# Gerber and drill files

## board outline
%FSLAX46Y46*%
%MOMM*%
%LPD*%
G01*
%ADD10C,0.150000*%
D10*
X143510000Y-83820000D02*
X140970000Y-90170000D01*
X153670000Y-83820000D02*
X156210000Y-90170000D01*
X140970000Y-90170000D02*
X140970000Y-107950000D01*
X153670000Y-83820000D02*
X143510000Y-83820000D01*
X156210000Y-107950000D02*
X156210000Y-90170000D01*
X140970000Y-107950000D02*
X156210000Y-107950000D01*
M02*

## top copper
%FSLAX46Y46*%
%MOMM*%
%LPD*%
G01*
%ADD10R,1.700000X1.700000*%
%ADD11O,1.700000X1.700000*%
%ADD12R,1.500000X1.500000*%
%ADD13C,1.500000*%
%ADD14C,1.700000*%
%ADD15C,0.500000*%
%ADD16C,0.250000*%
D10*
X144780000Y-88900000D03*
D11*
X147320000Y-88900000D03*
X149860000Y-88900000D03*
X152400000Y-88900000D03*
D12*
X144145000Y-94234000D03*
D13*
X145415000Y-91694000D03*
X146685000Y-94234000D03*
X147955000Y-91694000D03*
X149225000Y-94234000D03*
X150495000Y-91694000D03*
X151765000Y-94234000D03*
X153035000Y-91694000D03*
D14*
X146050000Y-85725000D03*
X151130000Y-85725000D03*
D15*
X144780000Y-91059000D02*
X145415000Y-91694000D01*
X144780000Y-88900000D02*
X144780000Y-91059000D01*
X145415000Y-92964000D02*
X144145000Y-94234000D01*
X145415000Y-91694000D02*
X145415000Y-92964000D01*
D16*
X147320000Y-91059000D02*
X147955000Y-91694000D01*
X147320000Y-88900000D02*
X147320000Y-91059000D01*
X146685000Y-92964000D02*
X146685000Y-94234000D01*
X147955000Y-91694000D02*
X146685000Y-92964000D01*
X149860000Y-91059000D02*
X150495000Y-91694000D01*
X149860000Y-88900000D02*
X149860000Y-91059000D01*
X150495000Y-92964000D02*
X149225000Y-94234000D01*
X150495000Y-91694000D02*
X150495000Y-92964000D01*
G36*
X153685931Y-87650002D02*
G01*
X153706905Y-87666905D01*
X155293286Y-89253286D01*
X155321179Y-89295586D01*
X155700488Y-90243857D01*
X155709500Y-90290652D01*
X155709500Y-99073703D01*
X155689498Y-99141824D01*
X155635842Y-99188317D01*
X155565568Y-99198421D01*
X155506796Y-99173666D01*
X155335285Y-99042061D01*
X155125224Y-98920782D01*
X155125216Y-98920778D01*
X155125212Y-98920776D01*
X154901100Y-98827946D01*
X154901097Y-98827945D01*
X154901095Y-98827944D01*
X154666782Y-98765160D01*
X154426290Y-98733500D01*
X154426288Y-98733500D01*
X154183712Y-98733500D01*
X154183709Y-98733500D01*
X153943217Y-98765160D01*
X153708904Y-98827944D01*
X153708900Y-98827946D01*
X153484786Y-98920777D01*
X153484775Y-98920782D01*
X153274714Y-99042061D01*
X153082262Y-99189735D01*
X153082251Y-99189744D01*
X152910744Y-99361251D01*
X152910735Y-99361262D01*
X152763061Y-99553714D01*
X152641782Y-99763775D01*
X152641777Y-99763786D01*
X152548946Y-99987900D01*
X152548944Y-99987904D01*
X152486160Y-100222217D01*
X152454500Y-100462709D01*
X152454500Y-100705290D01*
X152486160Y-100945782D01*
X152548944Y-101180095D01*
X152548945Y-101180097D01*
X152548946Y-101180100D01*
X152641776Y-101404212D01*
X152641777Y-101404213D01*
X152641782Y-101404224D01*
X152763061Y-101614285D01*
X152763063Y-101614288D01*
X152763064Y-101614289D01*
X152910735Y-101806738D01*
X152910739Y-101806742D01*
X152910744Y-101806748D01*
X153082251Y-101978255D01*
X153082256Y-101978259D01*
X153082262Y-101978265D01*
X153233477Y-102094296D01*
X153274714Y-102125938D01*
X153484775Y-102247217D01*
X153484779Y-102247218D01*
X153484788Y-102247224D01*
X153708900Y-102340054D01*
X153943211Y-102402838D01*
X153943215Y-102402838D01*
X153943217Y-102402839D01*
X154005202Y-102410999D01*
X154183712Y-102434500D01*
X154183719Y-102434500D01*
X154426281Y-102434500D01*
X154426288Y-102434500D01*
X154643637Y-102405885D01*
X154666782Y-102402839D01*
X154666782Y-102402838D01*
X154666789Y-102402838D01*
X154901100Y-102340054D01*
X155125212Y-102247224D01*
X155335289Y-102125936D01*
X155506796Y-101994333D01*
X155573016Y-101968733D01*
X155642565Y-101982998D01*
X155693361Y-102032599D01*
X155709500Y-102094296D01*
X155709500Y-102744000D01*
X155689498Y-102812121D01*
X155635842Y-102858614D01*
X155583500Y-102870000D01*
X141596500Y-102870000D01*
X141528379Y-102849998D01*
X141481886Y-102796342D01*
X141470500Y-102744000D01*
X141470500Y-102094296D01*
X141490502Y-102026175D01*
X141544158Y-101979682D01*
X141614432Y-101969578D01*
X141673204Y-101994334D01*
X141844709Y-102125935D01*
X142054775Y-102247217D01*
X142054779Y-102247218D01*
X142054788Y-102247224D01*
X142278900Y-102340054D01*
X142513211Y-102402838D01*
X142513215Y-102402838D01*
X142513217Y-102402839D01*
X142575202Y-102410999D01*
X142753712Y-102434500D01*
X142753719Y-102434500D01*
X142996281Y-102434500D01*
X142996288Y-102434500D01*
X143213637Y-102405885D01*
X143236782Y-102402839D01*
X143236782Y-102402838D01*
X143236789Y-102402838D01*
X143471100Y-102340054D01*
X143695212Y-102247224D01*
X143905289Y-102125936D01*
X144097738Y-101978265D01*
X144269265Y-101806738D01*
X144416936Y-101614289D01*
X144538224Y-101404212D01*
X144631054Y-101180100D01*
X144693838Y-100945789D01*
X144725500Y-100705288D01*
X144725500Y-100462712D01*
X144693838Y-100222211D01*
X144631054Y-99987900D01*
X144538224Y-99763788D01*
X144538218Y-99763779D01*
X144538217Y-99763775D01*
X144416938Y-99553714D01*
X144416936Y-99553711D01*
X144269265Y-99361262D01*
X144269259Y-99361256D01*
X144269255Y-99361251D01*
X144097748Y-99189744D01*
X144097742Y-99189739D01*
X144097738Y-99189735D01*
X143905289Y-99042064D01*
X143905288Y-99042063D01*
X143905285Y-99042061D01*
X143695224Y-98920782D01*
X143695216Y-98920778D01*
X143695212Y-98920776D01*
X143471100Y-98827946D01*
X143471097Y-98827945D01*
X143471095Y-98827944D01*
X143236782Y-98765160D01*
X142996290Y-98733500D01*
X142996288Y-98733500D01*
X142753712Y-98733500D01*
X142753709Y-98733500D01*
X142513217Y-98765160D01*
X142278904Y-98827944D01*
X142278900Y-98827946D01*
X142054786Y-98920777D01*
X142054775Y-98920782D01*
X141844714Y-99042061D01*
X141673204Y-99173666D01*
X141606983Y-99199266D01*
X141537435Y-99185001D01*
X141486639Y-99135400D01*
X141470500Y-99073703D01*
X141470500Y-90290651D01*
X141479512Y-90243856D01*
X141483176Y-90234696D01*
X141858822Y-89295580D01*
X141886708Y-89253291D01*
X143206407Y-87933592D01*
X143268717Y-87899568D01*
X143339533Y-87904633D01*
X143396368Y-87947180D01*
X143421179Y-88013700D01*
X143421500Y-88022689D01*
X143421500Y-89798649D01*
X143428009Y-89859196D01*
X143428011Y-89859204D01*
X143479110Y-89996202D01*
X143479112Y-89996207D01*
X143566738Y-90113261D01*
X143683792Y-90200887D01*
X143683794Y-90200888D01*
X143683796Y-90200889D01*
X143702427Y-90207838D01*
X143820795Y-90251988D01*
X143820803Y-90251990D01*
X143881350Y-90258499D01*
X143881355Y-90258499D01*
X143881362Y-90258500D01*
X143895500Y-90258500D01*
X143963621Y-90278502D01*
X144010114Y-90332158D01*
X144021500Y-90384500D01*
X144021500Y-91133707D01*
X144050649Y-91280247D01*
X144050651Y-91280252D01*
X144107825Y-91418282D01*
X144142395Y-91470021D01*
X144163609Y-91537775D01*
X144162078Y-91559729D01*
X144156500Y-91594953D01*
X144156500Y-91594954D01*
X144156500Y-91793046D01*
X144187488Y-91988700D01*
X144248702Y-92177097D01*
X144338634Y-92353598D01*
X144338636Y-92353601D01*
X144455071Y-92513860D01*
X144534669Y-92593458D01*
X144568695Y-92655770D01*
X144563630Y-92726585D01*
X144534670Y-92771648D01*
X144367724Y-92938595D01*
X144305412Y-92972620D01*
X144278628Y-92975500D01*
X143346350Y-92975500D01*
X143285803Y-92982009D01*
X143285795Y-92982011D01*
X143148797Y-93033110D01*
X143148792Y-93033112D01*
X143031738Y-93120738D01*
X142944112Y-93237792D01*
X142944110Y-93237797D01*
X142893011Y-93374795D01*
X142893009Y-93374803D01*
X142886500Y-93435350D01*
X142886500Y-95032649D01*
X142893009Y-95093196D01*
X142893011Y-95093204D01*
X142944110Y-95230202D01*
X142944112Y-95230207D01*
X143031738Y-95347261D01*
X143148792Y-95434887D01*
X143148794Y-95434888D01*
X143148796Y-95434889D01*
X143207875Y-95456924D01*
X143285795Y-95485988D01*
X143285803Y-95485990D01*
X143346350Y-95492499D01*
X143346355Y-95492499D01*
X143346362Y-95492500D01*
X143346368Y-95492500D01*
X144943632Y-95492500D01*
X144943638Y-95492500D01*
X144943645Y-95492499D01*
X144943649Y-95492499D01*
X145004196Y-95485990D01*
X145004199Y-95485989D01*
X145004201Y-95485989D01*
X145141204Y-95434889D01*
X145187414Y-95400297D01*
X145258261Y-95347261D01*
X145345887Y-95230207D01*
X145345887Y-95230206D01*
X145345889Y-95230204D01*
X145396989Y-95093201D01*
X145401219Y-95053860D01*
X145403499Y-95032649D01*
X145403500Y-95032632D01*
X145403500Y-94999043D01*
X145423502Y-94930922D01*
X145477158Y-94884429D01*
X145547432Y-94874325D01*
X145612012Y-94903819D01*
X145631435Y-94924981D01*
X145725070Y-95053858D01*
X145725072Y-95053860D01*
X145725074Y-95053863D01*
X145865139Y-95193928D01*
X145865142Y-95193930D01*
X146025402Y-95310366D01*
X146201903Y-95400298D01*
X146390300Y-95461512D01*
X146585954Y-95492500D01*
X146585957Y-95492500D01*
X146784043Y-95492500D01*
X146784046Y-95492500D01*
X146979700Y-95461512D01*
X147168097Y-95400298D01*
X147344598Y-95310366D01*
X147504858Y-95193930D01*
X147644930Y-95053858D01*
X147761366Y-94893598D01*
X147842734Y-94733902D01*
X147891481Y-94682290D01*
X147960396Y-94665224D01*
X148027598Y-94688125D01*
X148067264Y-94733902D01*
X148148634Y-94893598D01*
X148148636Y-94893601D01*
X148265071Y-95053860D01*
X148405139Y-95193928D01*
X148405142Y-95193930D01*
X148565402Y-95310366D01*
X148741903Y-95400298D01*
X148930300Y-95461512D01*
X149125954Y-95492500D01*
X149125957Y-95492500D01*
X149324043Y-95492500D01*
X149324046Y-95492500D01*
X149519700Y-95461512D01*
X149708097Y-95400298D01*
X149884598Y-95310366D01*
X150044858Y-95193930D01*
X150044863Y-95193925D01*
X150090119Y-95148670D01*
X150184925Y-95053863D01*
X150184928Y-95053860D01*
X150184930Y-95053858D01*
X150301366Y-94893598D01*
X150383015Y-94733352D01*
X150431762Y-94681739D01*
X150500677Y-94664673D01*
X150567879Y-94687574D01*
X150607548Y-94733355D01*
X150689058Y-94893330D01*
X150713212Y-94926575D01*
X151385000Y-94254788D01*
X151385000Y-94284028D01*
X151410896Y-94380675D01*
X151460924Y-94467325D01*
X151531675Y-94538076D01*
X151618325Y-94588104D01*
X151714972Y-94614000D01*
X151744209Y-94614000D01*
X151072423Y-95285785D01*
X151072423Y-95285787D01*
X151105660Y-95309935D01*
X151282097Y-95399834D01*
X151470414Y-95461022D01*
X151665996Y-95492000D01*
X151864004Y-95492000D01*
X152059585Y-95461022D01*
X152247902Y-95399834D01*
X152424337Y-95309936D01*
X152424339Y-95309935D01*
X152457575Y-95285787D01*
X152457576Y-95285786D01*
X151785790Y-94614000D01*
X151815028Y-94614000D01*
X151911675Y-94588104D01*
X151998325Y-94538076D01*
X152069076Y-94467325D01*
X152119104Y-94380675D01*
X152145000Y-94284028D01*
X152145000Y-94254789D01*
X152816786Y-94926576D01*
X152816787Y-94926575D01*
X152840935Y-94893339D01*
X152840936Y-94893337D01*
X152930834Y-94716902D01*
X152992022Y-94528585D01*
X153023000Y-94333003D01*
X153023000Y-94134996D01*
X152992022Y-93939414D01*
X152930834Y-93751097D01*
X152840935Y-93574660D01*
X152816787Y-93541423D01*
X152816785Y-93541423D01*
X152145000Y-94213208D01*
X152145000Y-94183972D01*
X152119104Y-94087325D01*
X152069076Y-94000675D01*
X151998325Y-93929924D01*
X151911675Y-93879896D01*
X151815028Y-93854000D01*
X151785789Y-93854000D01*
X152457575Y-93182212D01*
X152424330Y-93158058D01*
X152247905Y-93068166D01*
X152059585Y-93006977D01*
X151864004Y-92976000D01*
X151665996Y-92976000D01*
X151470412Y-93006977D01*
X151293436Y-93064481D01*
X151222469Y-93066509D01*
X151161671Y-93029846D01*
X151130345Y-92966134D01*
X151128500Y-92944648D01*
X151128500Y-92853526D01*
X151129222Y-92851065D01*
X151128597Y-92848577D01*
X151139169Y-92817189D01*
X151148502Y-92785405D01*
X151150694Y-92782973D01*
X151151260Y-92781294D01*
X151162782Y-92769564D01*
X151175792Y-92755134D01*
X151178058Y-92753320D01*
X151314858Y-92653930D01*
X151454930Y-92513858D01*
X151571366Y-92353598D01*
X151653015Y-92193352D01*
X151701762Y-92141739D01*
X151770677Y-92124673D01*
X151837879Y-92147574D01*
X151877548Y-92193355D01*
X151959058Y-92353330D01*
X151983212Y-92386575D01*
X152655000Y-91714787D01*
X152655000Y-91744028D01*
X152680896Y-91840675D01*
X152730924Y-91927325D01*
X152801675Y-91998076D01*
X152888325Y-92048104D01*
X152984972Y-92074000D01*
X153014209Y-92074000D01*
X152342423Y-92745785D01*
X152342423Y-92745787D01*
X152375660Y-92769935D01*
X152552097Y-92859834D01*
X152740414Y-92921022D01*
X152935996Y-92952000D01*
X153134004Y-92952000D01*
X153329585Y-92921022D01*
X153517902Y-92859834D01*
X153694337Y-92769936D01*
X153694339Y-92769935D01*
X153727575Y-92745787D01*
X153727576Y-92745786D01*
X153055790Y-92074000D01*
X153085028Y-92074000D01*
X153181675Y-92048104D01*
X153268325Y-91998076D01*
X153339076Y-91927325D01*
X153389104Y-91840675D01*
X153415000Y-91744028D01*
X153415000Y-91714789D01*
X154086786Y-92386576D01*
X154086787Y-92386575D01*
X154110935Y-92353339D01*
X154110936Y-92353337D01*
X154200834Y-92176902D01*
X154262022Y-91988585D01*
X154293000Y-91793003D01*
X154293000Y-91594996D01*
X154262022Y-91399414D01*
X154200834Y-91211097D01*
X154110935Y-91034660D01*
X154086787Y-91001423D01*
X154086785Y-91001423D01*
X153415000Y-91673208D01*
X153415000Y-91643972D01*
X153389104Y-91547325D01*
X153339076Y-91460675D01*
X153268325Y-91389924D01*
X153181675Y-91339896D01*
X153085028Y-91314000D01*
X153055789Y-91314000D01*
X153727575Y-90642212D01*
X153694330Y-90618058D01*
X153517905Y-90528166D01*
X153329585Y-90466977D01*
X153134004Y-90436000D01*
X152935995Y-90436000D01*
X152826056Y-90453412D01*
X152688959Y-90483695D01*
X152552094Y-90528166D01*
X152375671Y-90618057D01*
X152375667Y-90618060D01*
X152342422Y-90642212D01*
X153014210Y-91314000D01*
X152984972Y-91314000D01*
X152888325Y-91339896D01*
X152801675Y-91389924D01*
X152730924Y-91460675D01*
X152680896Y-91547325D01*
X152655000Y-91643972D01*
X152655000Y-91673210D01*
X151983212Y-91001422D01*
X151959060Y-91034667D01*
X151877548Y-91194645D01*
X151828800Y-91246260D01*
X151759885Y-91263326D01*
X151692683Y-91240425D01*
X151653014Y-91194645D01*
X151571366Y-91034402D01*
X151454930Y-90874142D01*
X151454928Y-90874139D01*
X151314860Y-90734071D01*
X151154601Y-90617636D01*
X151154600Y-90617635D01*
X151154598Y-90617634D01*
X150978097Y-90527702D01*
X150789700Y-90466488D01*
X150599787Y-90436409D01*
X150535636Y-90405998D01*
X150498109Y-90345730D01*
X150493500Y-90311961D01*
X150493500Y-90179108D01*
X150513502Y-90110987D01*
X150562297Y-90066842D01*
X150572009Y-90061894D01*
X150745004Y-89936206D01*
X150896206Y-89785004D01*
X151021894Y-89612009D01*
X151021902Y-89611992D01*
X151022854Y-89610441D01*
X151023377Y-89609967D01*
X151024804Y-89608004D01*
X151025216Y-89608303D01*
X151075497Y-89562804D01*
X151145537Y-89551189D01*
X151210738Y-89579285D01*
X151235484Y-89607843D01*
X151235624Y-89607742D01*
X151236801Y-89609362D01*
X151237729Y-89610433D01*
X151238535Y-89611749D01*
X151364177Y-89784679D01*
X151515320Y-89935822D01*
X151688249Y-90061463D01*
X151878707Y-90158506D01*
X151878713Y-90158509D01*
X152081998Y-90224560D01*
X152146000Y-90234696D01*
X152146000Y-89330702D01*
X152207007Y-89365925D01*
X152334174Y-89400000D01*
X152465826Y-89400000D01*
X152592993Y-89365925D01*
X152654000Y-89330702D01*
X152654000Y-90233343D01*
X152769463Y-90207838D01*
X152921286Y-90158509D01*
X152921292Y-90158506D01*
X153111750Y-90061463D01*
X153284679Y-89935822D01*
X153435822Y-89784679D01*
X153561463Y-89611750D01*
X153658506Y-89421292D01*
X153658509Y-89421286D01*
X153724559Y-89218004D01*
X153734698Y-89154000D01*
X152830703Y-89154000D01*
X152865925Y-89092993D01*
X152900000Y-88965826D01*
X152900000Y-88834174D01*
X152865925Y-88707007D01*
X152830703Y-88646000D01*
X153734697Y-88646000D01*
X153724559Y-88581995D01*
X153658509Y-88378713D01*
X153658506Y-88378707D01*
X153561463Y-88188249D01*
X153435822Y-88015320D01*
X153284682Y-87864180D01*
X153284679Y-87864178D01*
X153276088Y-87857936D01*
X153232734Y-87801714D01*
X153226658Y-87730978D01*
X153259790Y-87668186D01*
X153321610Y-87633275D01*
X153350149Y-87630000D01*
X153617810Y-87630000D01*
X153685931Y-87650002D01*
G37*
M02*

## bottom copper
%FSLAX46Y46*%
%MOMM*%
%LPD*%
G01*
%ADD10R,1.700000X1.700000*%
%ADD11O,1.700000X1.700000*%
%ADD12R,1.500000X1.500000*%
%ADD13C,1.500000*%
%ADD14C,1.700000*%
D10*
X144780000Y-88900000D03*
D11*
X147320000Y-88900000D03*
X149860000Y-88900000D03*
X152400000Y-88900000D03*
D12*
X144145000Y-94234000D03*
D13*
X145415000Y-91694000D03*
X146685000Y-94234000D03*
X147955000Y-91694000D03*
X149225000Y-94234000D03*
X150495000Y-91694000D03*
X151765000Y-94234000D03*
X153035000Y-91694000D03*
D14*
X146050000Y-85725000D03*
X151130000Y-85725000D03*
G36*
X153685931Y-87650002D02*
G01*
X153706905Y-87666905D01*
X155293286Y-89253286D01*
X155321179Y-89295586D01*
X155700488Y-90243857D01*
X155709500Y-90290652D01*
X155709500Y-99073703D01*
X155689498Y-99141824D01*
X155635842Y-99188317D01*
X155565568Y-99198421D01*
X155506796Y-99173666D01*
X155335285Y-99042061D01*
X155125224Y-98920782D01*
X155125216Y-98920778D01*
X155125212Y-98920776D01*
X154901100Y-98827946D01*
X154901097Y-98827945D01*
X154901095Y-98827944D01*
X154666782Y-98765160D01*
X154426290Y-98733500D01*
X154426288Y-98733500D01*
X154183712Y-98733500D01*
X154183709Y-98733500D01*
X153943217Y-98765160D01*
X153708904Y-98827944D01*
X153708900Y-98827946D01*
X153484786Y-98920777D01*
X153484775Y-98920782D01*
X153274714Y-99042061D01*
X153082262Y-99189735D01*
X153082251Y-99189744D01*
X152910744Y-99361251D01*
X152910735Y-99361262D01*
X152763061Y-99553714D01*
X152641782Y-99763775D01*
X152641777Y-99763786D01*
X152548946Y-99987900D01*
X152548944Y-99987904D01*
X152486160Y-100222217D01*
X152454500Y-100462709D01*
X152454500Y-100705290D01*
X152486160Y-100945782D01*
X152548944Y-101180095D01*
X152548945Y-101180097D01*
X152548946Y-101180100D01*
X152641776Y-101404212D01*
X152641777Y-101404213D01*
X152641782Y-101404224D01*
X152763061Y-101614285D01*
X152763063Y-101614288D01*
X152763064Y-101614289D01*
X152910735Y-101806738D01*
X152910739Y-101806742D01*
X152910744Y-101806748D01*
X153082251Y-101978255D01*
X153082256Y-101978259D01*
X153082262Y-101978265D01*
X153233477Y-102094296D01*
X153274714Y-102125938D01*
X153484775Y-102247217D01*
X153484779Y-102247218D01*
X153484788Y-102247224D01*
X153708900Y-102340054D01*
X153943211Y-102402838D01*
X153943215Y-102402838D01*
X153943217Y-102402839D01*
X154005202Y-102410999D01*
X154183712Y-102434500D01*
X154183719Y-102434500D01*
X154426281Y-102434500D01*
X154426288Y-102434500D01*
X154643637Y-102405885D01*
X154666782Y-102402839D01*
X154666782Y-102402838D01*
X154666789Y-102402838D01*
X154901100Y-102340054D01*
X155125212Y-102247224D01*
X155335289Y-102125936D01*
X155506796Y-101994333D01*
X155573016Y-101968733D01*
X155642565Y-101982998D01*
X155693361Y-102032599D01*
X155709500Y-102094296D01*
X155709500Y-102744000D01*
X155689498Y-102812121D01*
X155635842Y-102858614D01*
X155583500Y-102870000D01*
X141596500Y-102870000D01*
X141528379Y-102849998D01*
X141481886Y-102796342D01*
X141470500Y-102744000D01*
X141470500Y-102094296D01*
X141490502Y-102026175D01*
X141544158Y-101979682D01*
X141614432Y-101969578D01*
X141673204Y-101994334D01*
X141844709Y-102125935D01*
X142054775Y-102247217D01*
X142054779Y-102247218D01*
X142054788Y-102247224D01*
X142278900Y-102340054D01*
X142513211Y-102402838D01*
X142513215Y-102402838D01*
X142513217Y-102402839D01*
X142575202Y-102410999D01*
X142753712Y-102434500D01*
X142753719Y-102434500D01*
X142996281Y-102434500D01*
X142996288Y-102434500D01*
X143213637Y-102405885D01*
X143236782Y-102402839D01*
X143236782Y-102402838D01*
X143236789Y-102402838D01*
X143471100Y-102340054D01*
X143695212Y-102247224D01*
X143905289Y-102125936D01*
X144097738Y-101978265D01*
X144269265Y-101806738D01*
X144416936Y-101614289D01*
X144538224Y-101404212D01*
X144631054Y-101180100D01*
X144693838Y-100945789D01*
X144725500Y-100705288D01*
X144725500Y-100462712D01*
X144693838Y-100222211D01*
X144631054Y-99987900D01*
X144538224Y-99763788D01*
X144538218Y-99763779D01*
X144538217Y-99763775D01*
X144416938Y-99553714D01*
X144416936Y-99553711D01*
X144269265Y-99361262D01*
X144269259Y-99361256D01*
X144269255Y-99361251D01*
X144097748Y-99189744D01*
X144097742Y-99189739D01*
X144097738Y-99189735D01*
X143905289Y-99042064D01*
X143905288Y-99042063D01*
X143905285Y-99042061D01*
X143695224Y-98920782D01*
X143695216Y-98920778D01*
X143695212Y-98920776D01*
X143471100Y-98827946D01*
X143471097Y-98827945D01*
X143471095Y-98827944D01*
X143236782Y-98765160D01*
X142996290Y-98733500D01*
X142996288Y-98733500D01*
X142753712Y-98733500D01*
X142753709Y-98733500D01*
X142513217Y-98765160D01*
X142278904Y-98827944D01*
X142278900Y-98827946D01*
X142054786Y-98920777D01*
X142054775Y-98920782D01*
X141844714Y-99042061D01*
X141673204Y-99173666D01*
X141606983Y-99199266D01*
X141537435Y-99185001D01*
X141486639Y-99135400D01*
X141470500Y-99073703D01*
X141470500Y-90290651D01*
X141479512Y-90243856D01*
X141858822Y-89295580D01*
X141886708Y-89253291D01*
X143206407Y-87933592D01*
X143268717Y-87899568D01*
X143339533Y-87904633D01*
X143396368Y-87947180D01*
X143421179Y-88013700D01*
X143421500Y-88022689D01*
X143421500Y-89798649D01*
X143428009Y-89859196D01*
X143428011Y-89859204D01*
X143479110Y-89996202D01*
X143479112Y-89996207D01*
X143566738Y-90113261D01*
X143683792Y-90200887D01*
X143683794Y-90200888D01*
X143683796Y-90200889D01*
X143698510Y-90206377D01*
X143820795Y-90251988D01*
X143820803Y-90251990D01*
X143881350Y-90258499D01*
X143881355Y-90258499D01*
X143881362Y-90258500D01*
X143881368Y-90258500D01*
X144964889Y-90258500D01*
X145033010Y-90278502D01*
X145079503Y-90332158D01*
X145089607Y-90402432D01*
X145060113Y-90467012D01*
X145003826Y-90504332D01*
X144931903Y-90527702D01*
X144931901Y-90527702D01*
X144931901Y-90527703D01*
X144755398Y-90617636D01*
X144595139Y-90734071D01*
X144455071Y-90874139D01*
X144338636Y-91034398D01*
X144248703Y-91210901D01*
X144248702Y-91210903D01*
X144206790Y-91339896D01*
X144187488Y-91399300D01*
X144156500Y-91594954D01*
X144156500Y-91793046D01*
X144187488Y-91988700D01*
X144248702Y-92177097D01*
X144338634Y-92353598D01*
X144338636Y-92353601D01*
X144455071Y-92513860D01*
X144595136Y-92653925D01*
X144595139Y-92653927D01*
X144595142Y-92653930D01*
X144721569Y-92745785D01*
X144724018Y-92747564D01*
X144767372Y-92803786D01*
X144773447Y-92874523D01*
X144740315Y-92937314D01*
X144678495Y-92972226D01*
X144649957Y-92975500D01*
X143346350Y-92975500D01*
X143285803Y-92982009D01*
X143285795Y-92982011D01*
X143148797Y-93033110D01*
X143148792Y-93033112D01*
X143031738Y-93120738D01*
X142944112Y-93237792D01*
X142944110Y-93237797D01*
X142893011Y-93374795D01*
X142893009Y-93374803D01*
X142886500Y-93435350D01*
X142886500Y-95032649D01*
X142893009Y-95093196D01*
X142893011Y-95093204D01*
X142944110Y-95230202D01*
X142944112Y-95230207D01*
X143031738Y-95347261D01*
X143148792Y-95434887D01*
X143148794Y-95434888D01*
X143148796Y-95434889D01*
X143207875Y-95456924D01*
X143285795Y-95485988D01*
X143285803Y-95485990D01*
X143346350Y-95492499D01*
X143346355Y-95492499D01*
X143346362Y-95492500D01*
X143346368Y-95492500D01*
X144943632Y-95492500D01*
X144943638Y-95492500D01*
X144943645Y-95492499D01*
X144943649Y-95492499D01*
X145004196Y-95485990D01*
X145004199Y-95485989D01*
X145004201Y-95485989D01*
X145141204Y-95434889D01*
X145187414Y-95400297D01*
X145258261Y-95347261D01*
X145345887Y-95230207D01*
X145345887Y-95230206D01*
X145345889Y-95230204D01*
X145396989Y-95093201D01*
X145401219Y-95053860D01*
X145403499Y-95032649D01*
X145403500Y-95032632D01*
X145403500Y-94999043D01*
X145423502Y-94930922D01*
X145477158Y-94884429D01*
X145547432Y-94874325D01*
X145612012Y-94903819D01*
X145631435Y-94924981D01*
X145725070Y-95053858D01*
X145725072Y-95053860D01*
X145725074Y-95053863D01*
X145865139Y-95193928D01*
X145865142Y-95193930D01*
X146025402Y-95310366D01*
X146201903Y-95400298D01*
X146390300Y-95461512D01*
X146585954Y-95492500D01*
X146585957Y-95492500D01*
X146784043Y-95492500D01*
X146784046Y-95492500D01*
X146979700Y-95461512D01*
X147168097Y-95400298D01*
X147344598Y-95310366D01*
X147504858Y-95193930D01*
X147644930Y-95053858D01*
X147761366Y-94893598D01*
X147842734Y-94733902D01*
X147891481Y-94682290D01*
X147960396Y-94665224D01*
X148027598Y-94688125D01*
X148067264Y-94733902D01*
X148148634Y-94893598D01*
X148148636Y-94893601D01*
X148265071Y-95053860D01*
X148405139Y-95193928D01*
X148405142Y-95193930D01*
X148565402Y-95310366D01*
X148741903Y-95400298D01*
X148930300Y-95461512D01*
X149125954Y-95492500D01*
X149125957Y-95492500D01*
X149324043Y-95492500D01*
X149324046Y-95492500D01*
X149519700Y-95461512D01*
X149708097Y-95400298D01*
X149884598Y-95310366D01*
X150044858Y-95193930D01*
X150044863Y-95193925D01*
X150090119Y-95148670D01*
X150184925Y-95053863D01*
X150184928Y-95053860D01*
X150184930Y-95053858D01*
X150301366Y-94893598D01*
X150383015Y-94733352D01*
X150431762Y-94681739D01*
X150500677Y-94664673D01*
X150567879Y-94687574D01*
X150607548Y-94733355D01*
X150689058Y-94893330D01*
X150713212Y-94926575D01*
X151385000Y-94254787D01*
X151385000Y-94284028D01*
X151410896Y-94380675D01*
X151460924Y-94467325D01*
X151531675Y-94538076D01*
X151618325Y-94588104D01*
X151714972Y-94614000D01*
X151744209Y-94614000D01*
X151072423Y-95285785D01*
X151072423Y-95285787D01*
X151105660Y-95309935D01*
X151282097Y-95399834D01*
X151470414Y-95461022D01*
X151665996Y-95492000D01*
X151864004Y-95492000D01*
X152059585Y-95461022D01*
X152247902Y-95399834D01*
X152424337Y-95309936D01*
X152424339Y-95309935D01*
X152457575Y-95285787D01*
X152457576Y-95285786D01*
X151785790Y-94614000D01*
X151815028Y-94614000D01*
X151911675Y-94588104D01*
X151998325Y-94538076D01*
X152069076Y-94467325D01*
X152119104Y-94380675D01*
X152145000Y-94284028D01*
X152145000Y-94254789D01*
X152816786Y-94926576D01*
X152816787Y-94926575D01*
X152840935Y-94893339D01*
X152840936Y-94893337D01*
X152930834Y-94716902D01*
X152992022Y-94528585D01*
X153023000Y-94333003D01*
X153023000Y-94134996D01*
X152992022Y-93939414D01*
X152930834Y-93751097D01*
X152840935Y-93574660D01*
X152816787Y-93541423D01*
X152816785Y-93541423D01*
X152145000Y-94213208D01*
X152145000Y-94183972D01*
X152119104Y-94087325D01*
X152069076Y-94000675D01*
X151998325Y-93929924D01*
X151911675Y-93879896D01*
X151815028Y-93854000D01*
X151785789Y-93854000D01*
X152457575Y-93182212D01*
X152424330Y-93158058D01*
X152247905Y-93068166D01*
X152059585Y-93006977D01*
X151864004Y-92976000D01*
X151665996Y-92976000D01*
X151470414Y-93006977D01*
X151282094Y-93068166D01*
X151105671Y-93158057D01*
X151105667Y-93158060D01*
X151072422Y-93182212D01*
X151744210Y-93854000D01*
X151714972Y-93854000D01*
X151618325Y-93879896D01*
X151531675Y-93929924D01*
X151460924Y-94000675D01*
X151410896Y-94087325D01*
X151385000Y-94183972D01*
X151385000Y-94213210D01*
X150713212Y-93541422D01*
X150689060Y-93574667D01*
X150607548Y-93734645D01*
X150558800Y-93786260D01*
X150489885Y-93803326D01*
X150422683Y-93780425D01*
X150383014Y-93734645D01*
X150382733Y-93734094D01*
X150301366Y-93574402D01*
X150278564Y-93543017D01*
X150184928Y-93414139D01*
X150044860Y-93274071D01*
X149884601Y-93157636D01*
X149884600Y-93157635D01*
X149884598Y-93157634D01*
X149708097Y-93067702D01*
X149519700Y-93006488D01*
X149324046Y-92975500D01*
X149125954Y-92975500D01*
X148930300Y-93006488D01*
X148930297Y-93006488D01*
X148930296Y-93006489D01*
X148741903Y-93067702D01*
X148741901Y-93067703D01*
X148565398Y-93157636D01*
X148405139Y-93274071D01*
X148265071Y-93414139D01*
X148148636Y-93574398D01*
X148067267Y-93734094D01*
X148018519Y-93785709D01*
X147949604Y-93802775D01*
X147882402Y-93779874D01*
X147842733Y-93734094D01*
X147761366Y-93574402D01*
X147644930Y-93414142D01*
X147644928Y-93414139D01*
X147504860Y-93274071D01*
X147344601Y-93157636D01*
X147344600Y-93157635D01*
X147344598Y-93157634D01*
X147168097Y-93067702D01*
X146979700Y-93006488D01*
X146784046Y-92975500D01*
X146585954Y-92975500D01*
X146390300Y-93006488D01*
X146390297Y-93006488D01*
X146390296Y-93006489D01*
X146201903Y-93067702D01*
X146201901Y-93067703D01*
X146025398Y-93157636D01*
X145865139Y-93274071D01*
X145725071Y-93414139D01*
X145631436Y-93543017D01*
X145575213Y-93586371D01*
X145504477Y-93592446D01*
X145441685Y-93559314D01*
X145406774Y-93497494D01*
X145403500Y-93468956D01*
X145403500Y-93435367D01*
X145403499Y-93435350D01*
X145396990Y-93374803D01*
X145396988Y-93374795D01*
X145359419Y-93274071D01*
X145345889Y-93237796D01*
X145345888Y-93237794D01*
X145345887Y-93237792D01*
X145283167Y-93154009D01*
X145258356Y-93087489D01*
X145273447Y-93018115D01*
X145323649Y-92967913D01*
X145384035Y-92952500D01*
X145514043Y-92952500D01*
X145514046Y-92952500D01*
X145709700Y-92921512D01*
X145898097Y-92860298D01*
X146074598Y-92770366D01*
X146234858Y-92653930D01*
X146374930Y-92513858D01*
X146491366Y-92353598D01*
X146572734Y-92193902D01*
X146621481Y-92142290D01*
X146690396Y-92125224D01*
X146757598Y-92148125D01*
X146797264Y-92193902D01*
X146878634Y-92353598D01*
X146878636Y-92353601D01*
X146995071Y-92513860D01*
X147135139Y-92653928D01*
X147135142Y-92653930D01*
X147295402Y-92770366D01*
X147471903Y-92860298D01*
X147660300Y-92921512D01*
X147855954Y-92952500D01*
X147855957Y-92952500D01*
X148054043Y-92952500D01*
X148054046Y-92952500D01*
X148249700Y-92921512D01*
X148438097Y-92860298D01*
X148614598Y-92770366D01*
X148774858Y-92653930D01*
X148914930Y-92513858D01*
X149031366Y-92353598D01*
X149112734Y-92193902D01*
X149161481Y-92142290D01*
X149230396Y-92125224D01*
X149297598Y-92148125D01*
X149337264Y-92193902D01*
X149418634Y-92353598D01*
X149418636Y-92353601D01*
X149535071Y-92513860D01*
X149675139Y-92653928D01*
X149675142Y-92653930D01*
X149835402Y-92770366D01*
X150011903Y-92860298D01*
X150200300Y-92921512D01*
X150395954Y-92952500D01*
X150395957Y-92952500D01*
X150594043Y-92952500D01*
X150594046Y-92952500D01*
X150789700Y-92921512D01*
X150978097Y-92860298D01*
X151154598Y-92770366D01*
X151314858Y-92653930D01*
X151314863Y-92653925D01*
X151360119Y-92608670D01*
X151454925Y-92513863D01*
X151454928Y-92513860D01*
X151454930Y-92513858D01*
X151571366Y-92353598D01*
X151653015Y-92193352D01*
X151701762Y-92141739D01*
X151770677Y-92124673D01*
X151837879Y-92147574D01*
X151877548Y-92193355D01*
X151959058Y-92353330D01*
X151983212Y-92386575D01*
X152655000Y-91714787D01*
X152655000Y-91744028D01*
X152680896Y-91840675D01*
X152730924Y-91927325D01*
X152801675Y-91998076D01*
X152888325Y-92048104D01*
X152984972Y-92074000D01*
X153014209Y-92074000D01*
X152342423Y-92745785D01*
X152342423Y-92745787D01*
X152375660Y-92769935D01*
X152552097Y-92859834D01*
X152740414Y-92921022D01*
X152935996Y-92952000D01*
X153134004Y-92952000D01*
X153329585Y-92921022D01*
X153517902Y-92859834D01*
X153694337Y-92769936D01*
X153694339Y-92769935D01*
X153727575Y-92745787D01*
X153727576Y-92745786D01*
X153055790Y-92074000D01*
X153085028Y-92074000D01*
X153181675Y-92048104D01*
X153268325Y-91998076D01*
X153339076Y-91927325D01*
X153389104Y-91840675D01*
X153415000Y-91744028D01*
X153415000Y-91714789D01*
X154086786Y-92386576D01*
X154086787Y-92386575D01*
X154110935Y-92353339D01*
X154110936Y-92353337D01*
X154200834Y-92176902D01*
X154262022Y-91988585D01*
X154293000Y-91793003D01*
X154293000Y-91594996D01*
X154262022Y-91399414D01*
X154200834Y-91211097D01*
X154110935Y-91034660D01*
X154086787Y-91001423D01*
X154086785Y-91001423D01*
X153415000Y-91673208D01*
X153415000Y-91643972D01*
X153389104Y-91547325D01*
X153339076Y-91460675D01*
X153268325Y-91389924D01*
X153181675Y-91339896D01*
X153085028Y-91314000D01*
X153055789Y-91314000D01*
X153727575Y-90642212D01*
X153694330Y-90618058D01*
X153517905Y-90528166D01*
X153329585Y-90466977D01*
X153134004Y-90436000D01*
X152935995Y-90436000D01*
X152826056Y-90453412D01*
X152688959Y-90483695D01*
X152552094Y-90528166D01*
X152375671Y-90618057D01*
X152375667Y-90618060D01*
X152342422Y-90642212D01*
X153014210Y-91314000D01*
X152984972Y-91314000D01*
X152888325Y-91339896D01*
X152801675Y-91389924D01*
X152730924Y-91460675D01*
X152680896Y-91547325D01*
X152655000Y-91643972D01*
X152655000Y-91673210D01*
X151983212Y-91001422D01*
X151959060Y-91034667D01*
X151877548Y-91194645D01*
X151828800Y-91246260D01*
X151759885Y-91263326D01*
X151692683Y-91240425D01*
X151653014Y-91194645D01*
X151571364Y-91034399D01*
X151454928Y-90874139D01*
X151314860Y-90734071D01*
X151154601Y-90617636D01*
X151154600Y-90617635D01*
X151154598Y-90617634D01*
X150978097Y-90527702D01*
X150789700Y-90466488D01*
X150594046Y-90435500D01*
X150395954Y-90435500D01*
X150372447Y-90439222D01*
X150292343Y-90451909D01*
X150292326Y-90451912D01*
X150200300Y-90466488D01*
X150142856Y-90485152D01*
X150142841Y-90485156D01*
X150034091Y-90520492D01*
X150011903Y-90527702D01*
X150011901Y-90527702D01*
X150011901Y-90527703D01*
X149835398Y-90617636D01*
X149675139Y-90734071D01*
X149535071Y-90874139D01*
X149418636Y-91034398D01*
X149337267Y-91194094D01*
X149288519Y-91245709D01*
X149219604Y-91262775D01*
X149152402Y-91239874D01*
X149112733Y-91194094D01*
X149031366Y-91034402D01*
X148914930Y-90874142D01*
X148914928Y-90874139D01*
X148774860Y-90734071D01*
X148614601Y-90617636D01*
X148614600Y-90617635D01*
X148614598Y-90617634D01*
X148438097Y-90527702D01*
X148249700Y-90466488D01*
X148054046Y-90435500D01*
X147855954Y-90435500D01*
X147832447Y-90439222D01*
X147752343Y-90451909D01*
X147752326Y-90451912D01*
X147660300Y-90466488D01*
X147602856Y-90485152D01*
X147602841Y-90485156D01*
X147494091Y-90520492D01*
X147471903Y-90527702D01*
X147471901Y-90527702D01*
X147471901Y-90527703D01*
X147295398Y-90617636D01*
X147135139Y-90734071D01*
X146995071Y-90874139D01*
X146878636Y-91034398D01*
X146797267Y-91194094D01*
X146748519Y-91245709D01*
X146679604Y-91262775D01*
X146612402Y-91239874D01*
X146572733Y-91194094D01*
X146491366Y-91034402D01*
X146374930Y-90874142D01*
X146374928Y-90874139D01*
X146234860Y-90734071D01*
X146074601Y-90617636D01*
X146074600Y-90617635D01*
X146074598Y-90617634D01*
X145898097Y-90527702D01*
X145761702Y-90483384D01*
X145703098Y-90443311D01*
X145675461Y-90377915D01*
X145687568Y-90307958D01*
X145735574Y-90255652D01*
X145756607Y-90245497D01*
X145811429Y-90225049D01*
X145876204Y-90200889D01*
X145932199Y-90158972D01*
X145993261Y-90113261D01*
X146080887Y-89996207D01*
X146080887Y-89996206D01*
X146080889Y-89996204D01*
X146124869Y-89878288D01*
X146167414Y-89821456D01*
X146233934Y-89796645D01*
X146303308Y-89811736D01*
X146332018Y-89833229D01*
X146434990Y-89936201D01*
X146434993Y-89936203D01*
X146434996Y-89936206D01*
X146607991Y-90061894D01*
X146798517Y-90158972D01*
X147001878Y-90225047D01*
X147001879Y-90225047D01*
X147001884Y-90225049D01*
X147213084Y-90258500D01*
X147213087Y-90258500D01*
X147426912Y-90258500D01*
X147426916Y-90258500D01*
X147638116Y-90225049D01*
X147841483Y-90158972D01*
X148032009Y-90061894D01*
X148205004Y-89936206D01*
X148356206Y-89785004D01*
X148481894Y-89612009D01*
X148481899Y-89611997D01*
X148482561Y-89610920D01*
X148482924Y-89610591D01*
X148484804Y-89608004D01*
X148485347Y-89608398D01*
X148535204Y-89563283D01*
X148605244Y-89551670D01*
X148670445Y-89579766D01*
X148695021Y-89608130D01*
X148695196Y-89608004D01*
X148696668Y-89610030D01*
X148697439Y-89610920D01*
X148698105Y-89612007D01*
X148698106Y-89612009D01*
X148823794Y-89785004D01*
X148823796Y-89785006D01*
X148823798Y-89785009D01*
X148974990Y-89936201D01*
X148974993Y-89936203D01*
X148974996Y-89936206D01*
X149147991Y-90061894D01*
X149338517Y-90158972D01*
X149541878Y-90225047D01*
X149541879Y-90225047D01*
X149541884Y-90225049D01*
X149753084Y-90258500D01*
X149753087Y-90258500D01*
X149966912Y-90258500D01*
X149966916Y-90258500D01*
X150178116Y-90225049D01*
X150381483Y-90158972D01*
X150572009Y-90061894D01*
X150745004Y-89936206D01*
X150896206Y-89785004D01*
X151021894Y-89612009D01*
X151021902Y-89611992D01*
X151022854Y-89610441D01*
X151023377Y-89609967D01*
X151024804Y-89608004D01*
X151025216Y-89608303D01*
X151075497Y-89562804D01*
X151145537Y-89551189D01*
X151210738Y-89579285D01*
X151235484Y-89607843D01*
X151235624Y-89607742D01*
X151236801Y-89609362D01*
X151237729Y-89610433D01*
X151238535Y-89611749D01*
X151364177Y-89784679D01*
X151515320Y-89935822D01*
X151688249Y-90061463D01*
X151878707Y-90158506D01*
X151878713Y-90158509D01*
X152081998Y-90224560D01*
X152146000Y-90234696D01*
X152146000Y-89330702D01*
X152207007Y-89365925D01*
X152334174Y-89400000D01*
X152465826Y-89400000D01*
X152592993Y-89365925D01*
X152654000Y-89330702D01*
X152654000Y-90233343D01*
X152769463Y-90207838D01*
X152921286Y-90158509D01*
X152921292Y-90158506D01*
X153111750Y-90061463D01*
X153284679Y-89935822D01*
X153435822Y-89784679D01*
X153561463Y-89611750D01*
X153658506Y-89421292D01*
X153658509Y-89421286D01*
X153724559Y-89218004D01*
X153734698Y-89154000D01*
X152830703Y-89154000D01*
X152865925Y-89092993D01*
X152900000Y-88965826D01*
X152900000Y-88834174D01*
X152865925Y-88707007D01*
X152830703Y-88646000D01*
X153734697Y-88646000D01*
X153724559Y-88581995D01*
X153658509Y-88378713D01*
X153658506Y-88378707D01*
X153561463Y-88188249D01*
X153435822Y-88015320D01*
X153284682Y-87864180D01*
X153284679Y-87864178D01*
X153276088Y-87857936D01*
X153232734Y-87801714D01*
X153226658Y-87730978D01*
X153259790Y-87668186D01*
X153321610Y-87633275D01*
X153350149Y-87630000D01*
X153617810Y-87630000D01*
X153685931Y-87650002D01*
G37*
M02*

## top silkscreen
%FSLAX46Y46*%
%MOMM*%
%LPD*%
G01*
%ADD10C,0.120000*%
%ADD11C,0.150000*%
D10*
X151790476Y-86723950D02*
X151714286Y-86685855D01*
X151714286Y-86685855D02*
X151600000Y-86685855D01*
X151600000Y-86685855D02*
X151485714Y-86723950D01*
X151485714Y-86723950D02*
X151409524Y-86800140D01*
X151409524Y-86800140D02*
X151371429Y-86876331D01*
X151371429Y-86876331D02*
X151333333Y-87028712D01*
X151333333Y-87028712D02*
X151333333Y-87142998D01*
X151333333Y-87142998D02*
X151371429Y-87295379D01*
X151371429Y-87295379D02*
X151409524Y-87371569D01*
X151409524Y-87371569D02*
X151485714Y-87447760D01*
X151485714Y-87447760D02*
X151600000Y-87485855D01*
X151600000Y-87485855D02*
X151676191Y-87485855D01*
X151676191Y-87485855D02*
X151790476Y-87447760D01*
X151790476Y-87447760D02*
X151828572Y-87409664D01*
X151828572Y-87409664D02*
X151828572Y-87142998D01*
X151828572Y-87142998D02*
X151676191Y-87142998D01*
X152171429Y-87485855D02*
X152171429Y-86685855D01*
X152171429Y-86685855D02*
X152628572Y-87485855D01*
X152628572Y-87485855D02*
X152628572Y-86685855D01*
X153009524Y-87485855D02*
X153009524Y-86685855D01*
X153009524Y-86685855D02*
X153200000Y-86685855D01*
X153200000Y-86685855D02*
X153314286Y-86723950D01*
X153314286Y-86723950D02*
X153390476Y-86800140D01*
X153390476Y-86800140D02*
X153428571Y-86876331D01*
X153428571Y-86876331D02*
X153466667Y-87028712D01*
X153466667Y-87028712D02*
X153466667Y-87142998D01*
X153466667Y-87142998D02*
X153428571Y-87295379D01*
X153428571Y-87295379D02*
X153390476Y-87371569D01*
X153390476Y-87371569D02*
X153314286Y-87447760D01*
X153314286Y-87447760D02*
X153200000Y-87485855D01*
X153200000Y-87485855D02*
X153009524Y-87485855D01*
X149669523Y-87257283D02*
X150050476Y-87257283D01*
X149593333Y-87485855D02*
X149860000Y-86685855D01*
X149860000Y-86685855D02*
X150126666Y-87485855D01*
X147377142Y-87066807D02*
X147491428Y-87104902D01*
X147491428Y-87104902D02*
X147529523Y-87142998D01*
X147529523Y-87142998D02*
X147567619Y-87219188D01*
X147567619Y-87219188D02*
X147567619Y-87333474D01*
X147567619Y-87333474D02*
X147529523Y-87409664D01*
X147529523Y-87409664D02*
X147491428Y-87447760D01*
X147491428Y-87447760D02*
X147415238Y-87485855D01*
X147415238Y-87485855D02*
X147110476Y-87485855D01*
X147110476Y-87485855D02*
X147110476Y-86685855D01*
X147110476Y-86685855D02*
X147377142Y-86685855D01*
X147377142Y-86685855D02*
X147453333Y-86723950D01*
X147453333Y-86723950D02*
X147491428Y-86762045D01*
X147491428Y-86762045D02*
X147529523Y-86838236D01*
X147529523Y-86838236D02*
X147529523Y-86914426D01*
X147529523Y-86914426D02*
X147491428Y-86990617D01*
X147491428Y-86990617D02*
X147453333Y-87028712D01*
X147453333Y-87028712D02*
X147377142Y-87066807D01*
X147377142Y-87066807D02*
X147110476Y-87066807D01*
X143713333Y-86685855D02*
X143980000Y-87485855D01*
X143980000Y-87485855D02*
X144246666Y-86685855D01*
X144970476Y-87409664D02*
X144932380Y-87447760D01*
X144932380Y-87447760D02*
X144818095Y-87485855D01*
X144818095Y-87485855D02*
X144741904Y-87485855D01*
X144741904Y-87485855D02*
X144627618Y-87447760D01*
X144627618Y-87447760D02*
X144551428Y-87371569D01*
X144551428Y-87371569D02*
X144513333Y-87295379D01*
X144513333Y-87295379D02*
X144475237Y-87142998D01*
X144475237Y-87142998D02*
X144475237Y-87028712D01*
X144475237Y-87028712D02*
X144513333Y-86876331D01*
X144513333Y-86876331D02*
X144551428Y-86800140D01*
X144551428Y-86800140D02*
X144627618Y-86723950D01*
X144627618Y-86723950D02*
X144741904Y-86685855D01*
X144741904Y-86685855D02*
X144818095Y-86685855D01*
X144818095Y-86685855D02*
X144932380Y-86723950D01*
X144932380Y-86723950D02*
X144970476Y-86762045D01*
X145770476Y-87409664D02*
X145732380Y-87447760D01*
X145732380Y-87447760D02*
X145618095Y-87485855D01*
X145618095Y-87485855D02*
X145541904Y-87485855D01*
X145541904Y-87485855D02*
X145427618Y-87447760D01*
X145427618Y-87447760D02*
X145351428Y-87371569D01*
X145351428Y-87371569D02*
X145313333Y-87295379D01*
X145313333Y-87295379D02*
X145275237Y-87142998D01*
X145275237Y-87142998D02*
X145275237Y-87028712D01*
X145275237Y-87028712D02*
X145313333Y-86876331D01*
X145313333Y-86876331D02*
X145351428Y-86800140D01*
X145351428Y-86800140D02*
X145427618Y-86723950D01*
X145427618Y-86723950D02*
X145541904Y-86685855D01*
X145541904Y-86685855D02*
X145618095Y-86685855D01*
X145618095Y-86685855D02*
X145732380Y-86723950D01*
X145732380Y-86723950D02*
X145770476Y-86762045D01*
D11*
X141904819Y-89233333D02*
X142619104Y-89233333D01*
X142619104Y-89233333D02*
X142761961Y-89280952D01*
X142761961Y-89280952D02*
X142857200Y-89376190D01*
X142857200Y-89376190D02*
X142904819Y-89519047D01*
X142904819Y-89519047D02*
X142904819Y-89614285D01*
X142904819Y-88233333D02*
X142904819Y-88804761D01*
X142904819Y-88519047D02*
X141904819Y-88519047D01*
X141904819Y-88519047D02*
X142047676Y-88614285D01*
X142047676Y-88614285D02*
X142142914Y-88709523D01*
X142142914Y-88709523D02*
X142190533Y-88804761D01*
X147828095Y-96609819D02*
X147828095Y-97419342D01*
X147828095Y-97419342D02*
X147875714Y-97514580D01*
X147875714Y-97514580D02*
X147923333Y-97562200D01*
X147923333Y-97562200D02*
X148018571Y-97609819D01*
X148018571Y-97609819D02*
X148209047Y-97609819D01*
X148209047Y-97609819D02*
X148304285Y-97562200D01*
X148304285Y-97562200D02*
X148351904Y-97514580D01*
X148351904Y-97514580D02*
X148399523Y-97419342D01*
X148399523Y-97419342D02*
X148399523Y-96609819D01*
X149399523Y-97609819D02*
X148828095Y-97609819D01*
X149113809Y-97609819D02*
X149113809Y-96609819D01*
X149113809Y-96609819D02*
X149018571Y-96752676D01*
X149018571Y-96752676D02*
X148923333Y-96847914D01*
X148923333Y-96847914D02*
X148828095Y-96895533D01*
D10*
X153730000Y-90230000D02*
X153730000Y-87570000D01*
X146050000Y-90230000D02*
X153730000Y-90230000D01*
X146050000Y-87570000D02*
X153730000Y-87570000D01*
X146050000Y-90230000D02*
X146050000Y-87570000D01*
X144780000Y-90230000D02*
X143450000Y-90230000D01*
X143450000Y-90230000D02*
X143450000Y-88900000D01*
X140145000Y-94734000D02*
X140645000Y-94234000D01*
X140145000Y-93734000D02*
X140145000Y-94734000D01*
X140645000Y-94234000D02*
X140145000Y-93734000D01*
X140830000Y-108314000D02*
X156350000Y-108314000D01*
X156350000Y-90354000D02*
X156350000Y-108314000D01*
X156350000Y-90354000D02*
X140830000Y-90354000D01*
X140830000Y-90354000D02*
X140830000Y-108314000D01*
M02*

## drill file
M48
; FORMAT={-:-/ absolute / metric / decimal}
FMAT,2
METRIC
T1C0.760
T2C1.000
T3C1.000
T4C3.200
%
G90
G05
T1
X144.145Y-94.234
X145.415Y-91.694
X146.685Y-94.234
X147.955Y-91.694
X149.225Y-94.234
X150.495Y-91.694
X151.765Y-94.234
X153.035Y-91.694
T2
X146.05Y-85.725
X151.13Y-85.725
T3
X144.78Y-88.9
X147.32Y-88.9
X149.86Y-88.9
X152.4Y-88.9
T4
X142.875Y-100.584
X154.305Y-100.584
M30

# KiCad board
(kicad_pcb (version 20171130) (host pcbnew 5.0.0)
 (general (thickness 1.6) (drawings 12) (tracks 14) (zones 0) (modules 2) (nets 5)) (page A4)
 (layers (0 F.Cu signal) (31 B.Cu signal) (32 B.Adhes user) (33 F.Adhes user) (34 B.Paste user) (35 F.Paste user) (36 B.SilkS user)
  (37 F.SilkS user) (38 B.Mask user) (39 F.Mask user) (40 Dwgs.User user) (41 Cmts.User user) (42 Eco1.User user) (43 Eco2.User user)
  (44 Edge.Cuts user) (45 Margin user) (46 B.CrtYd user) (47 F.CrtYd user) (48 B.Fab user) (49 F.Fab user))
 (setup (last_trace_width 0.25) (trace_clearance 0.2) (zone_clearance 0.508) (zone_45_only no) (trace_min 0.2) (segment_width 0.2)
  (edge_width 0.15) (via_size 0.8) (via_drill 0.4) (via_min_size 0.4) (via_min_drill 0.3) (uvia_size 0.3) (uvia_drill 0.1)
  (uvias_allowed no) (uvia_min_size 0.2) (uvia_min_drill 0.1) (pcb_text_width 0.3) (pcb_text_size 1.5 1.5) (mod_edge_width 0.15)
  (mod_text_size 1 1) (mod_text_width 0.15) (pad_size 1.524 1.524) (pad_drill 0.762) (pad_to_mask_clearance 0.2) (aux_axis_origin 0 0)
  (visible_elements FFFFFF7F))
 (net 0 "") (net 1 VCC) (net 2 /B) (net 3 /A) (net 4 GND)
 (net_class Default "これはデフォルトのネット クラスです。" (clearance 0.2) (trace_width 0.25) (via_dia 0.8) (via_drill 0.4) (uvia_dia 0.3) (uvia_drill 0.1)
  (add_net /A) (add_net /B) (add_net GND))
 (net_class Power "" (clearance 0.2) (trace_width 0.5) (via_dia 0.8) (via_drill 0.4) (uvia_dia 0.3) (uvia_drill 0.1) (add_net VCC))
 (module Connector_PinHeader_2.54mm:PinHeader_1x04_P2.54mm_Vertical (layer F.Cu) (at 144.78 88.9 90)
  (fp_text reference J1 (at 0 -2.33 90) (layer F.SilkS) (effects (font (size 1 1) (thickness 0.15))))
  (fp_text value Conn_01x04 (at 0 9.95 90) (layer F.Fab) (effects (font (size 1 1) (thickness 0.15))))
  (fp_line (start -1.33 8.95) (end 1.33 8.95) (layer F.SilkS) (width 0.12))
  (fp_line (start -1.33 1.27) (end -1.33 8.95) (layer F.SilkS) (width 0.12))
  (fp_line (start 1.33 1.27) (end 1.33 8.95) (layer F.SilkS) (width 0.12))
  (fp_line (start -1.33 1.27) (end 1.33 1.27) (layer F.SilkS) (width 0.12))
  (fp_line (start -1.33 0) (end -1.33 -1.33) (layer F.SilkS) (width 0.12))
  (fp_line (start -1.33 -1.33) (end 0 -1.33) (layer F.SilkS) (width 0.12))
  (pad 1 thru_hole rect (at 0 0 90) (size 1.7 1.7) (drill 1) (layers *.Cu *.Mask) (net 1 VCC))
  (pad 2 thru_hole oval (at 0 2.54 90) (size 1.7 1.7) (drill 1) (layers *.Cu *.Mask) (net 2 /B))
  (pad 3 thru_hole oval (at 0 5.08 90) (size 1.7 1.7) (drill 1) (layers *.Cu *.Mask) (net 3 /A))
  (pad 4 thru_hole oval (at 0 7.62 90) (size 1.7 1.7) (drill 1) (layers *.Cu *.Mask) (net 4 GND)))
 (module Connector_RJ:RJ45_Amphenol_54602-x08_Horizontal (layer F.Cu) (at 144.145 94.234)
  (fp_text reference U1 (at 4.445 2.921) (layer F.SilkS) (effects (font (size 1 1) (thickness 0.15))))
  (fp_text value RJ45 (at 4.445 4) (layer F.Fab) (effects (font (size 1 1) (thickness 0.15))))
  (fp_line (start -4 0.5) (end -3.5 0) (layer F.SilkS) (width 0.12))
  (fp_line (start -4 -0.5) (end -4 0.5) (layer F.SilkS) (width 0.12))
  (fp_line (start -3.5 0) (end -4 -0.5) (layer F.SilkS) (width 0.12))
  (fp_line (start -3.315 14.08) (end 12.205 14.08) (layer F.SilkS) (width 0.12))
  (fp_line (start 12.205 -3.88) (end 12.205 14.08) (layer F.SilkS) (width 0.12))
  (fp_line (start 12.205 -3.88) (end -3.315 -3.88) (layer F.SilkS) (width 0.12))
  (fp_line (start -3.315 -3.88) (end -3.315 14.08) (layer F.SilkS) (width 0.12))
  (pad "" np_thru_hole circle (at 10.16 6.35) (size 3.2 3.2) (drill 3.2) (layers *.Cu *.Mask))
  (pad "" np_thru_hole circle (at -1.27 6.35) (size 3.2 3.2) (drill 3.2) (layers *.Cu *.Mask))
  (pad 1 thru_hole rect (at 0 0) (size 1.5 1.5) (drill 0.76) (layers *.Cu *.Mask) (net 1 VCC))
  (pad 2 thru_hole circle (at 1.27 -2.54) (size 1.5 1.5) (drill 0.76) (layers *.Cu *.Mask) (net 1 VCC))
  (pad 3 thru_hole circle (at 2.54 0) (size 1.5 1.5) (drill 0.76) (layers *.Cu *.Mask) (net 2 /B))
  (pad 4 thru_hole circle (at 3.81 -2.54) (size 1.5 1.5) (drill 0.76) (layers *.Cu *.Mask) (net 2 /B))
  (pad 5 thru_hole circle (at 5.08 0) (size 1.5 1.5) (drill 0.76) (layers *.Cu *.Mask) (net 3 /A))
  (pad 6 thru_hole circle (at 6.35 -2.54) (size 1.5 1.5) (drill 0.76) (layers *.Cu *.Mask) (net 3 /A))
  (pad 7 thru_hole circle (at 7.62 0) (size 1.5 1.5) (drill 0.76) (layers *.Cu *.Mask) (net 4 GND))
  (pad 8 thru_hole circle (at 8.89 -2.54) (size 1.5 1.5) (drill 0.76) (layers *.Cu *.Mask) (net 4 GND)))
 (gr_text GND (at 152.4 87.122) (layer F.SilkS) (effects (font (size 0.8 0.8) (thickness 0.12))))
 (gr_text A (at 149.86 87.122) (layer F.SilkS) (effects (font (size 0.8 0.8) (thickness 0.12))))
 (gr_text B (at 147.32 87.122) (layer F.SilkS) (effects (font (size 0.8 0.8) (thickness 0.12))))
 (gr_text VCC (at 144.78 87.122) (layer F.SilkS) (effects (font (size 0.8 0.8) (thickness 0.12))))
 (gr_line (start 143.51 83.82) (end 140.97 90.17) (layer Edge.Cuts) (width 0.15))
 (gr_line (start 153.67 83.82) (end 156.21 90.17) (layer Edge.Cuts) (width 0.15))
 (gr_line (start 140.97 90.17) (end 140.97 107.95) (layer Edge.Cuts) (width 0.15))
 (gr_line (start 153.67 83.82) (end 143.51 83.82) (layer Edge.Cuts) (width 0.15))
 (gr_line (start 156.21 107.95) (end 156.21 90.17) (layer Edge.Cuts) (width 0.15))
 (gr_line (start 140.97 107.95) (end 156.21 107.95) (layer Edge.Cuts) (width 0.15))
 (via (at 146.05 85.725) (size 1.7) (drill 1) (layers F.Cu B.Cu) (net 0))
 (via (at 151.13 85.725) (size 1.7) (drill 1) (layers F.Cu B.Cu) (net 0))
 (segment (start 144.78 91.059) (end 145.415 91.694) (width 0.5) (layer F.Cu) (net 1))
 (segment (start 144.78 88.9) (end 144.78 91.059) (width 0.5) (layer F.Cu) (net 1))
 (segment (start 145.415 92.964) (end 144.145 94.234) (width 0.5) (layer F.Cu) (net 1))
 (segment (start 145.415 91.694) (end 145.415 92.964) (width 0.5) (layer F.Cu) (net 1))
 (segment (start 147.32 91.059) (end 147.955 91.694) (width 0.25) (layer F.Cu) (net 2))
 (segment (start 147.32 88.9) (end 147.32 91.059) (width 0.25) (layer F.Cu) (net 2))
 (segment (start 146.685 92.964) (end 146.685 94.234) (width 0.25) (layer F.Cu) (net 2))
 (segment (start 147.955 91.694) (end 146.685 92.964) (width 0.25) (layer F.Cu) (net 2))
 (segment (start 149.86 91.059) (end 150.495 91.694) (width 0.25) (layer F.Cu) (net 3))
 (segment (start 149.86 88.9) (end 149.86 91.059) (width 0.25) (layer F.Cu) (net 3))
 (segment (start 150.495 92.964) (end 149.225 94.234) (width 0.25) (layer F.Cu) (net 3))
 (segment (start 150.495 91.694) (end 150.495 92.964) (width 0.25) (layer F.Cu) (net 3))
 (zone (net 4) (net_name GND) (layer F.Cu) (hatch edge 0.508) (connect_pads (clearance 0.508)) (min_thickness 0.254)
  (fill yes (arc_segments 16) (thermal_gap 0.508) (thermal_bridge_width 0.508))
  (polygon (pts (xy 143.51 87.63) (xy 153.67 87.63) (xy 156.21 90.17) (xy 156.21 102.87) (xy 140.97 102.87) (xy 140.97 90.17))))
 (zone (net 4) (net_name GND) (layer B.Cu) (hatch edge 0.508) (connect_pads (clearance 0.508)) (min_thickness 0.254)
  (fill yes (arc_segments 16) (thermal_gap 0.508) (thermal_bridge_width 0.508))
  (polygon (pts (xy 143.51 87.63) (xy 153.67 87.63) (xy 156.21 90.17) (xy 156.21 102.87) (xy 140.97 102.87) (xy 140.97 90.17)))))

